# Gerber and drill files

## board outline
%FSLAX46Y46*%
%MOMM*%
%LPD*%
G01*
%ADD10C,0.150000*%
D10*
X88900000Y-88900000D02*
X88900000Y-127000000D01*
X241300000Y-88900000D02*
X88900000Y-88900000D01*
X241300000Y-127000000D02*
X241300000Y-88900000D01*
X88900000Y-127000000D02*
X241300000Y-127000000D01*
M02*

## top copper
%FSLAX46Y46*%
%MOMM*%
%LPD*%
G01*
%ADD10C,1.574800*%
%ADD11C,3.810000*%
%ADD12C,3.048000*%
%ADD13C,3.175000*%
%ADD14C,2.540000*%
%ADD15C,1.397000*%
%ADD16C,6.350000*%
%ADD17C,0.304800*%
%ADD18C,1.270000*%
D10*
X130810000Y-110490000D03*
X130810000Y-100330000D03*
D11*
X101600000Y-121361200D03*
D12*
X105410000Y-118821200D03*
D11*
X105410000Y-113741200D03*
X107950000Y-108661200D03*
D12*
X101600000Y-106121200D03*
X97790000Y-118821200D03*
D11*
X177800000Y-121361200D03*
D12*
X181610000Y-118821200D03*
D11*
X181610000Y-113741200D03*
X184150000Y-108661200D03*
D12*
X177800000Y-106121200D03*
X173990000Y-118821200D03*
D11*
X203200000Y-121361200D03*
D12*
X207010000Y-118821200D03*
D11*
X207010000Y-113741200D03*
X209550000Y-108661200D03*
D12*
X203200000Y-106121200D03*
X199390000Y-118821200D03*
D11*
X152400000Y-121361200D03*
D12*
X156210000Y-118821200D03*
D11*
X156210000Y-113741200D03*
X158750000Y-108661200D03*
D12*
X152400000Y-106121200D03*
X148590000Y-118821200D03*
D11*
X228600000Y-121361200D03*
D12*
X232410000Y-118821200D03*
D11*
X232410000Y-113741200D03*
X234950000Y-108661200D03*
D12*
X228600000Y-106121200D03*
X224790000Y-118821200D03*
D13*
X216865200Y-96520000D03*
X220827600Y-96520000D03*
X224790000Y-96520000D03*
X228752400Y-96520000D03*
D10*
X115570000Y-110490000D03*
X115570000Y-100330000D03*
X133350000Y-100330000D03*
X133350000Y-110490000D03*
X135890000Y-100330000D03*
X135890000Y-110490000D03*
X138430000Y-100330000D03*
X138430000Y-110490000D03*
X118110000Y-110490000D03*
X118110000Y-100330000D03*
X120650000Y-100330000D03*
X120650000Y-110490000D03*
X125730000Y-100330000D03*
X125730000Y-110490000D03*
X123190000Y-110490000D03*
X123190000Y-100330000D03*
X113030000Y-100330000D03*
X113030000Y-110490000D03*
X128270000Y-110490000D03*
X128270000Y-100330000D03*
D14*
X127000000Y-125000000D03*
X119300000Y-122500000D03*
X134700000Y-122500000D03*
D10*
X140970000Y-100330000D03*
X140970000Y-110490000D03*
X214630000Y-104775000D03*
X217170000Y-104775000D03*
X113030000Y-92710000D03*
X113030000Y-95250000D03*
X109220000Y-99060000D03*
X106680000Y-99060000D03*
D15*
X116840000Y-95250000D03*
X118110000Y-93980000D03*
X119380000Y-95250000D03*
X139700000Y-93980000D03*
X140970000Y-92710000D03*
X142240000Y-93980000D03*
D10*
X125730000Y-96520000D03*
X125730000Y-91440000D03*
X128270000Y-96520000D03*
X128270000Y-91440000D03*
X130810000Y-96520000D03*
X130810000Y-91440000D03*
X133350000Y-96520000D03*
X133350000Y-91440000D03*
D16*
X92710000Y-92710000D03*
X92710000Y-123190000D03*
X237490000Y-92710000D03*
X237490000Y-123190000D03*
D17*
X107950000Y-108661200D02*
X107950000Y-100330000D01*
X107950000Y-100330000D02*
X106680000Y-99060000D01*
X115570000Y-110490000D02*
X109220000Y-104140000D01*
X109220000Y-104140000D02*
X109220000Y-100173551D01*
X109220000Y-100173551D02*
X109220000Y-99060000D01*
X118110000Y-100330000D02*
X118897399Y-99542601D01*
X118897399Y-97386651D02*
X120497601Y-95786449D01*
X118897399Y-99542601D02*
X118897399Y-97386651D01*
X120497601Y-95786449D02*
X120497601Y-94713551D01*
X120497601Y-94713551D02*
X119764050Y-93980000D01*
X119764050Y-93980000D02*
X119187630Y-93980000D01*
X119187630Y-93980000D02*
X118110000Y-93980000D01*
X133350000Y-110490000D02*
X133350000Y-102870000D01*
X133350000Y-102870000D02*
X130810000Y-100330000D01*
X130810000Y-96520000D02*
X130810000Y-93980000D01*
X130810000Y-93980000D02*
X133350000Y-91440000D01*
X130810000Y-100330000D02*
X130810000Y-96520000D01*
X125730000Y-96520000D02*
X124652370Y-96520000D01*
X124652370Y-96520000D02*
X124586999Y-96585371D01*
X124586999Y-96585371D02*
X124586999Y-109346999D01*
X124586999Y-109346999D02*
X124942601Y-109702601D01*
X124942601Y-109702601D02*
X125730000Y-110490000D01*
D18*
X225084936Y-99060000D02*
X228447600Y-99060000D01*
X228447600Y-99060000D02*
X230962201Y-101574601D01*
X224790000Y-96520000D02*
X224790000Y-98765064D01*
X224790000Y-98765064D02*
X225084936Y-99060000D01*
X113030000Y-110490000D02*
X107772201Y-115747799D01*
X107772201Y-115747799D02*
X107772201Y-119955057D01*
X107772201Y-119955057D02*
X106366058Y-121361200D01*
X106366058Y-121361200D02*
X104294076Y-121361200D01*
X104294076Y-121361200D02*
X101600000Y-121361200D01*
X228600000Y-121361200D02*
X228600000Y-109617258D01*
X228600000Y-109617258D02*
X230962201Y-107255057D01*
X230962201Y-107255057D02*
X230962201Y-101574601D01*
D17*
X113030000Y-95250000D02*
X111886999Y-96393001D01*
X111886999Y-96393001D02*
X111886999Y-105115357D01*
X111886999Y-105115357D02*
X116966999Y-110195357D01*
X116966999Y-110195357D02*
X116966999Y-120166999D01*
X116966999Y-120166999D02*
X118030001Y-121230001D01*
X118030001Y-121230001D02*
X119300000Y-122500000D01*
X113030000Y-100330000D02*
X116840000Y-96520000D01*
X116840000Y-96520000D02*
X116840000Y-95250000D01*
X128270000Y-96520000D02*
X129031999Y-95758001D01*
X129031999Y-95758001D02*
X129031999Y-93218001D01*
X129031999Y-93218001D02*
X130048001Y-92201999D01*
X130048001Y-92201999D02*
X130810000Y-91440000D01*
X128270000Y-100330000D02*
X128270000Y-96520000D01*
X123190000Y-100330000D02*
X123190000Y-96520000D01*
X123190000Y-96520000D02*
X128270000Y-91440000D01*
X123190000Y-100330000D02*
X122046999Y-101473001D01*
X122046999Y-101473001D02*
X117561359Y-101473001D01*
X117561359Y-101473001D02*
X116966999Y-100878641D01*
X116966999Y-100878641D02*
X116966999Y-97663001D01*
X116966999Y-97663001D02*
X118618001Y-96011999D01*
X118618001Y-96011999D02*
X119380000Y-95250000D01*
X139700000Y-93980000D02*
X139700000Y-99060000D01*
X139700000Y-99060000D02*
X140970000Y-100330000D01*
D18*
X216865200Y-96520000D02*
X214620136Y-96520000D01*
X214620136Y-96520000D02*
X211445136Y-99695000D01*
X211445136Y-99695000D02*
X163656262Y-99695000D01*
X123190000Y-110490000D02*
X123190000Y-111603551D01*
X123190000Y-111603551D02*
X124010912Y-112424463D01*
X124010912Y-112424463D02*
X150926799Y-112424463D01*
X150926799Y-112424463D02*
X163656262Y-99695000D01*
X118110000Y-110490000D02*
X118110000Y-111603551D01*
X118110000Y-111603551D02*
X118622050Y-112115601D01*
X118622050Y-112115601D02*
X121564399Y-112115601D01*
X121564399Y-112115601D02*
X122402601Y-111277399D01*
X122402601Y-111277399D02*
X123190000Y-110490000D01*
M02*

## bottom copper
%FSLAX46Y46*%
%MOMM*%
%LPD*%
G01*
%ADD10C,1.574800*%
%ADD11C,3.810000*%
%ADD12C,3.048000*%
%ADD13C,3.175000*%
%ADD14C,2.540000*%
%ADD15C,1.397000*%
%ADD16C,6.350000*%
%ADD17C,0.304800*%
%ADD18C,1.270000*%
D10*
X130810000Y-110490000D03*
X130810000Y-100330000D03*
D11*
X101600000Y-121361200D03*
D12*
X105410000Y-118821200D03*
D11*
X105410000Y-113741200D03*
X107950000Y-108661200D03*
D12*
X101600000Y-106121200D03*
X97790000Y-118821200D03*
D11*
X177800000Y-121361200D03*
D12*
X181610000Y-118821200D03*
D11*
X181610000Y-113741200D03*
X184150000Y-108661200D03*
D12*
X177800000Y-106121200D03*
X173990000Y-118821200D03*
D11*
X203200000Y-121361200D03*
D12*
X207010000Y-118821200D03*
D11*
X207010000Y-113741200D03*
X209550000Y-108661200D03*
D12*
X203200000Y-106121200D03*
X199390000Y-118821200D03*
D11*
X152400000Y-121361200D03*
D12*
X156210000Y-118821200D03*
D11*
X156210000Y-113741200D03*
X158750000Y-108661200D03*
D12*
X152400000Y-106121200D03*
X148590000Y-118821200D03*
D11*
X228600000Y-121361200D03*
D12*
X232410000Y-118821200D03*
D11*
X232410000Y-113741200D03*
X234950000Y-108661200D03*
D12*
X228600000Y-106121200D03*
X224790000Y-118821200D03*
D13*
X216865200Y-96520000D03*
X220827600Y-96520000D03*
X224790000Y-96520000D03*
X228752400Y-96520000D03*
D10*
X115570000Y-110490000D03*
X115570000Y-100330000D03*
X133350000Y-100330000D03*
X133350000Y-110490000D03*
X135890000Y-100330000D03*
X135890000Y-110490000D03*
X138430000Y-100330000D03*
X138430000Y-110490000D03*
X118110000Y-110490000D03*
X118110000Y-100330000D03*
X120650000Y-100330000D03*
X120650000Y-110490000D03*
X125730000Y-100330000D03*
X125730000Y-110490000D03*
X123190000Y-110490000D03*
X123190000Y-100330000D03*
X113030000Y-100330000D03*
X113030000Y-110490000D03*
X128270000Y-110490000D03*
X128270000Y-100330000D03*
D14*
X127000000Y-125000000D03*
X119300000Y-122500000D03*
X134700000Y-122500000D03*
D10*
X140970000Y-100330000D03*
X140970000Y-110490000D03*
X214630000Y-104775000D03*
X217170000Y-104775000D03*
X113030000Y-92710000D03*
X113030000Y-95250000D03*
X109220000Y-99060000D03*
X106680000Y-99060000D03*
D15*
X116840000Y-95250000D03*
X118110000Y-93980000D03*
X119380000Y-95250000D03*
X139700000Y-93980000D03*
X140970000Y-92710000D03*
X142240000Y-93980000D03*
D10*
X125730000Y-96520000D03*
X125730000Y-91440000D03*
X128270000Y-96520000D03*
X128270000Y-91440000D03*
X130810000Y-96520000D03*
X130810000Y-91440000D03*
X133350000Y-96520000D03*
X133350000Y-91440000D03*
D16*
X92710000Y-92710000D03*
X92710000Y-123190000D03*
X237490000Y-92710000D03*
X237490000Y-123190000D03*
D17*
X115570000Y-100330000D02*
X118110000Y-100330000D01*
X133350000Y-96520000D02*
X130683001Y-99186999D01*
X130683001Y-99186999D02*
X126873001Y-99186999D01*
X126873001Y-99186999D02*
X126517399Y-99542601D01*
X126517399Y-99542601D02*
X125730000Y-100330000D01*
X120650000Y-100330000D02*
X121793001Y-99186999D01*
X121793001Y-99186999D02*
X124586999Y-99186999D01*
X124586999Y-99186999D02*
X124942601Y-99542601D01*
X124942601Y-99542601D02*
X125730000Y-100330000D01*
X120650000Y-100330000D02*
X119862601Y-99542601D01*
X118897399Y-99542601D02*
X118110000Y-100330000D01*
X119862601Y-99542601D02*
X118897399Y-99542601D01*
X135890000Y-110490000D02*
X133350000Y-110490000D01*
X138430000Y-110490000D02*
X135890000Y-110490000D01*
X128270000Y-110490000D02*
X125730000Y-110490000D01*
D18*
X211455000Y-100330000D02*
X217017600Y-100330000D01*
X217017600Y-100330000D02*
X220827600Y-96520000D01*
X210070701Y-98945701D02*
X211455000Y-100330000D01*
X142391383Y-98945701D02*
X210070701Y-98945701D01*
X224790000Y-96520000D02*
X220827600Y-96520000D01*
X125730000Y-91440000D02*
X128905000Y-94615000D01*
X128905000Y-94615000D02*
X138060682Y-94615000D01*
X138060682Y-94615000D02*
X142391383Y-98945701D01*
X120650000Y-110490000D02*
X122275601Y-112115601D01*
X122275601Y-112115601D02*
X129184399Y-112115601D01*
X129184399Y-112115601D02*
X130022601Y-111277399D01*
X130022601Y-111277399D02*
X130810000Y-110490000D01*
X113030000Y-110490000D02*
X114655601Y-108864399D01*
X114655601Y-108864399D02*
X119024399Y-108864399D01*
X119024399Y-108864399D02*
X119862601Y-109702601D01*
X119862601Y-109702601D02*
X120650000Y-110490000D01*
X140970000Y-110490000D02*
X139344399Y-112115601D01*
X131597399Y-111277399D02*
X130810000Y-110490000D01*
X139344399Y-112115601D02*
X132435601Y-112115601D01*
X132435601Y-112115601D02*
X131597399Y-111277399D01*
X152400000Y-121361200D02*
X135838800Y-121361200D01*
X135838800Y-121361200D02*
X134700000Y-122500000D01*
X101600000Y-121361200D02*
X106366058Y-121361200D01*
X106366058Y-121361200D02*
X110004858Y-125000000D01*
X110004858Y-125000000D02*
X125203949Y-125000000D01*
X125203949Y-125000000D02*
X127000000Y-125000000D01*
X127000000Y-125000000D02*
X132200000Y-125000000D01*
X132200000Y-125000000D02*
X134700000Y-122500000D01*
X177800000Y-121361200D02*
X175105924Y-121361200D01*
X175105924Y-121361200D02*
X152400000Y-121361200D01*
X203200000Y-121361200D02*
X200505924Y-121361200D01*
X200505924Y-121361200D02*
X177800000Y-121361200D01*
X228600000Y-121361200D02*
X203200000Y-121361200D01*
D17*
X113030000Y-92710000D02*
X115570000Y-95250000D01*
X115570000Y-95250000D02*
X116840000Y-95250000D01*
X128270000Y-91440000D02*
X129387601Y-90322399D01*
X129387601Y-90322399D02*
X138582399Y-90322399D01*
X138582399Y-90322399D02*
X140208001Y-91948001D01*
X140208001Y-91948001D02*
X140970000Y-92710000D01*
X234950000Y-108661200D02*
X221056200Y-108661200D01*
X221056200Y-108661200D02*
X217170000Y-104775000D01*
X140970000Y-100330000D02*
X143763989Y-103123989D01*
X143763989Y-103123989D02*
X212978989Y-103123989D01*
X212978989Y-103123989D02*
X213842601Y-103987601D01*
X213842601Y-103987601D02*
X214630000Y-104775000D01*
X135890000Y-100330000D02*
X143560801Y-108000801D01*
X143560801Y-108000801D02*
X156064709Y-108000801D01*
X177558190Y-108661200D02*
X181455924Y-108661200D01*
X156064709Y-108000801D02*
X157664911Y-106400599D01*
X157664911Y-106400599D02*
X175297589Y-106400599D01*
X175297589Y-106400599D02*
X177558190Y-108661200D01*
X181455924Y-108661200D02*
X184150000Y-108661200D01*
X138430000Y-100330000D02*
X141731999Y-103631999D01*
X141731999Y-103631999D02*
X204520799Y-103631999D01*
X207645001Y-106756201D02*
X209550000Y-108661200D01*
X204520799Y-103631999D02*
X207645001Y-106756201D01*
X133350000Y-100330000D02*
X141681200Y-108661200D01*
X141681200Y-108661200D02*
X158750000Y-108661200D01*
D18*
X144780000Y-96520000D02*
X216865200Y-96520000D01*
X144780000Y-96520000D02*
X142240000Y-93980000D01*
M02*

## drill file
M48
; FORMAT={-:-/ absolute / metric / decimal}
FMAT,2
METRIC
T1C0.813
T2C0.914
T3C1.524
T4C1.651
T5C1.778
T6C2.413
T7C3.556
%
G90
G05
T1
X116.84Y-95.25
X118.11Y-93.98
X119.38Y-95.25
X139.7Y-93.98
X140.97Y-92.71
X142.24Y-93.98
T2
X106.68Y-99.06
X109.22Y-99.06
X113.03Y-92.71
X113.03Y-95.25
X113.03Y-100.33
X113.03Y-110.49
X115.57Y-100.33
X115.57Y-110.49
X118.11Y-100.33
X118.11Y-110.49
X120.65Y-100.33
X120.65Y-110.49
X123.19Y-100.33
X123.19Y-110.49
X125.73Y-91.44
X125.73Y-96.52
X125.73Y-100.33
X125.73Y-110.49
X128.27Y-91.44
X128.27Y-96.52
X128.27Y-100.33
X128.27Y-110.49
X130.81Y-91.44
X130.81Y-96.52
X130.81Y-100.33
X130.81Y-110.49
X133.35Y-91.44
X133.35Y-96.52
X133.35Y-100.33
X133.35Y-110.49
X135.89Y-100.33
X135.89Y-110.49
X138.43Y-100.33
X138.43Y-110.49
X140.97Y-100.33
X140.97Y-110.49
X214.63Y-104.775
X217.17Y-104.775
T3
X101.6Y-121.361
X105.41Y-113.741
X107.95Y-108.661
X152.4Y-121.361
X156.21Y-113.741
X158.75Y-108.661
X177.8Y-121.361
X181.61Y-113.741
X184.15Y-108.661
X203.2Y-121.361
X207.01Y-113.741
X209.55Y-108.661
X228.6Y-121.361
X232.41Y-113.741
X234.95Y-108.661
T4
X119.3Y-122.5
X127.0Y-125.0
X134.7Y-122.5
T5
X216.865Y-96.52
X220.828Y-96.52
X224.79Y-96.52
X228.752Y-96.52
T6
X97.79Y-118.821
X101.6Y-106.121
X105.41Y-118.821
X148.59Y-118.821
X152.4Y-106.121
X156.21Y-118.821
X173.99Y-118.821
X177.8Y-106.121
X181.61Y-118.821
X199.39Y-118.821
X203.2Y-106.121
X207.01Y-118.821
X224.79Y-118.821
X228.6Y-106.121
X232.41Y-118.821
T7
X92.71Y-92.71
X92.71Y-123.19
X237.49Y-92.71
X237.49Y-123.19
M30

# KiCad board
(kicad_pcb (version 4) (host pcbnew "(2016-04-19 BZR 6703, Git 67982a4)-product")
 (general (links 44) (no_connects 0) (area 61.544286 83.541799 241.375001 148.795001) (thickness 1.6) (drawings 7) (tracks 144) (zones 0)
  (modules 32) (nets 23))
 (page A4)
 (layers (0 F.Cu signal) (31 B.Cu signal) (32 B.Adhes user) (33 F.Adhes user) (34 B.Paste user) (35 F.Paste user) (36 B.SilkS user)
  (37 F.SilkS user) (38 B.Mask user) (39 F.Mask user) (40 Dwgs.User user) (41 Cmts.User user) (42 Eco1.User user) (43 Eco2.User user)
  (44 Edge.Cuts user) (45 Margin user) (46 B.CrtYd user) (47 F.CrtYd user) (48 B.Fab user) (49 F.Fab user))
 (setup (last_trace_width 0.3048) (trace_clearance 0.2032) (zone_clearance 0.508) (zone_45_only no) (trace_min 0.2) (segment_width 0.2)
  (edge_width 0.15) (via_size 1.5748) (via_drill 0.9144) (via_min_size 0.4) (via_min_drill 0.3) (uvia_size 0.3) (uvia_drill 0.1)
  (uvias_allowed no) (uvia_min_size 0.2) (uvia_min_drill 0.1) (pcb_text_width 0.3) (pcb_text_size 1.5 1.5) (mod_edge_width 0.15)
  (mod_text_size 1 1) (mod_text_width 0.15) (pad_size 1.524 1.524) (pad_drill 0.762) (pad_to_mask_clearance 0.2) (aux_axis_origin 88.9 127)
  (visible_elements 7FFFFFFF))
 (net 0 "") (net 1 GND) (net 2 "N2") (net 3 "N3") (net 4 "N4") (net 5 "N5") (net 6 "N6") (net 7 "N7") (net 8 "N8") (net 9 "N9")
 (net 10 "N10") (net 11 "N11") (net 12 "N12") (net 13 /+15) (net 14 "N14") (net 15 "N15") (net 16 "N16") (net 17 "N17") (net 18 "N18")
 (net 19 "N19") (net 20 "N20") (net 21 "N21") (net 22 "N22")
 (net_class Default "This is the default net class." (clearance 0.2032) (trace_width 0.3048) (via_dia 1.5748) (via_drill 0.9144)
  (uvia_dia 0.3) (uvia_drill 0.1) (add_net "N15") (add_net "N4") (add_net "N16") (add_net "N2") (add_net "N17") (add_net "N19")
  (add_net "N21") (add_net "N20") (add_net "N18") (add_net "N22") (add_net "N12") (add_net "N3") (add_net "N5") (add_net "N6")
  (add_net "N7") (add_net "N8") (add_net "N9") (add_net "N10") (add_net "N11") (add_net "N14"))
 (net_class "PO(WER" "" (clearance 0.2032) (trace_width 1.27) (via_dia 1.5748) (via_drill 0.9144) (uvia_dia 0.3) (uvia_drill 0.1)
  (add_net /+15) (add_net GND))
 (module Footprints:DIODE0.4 (layer F.Cu) (at 130.81 105.41 90)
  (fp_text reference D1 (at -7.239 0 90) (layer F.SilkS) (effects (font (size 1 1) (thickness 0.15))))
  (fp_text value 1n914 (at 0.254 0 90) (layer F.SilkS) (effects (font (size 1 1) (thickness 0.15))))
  (pad 1 thru_hole circle (at -5.08 0 90) (size 1.5748 1.5748) (drill 0.9144) (layers *.Cu *.Mask F.SilkS) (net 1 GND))
  (pad 2 thru_hole circle (at 5.08 0 90) (size 1.5748 1.5748) (drill 0.9144) (layers *.Cu *.Mask F.SilkS) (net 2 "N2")))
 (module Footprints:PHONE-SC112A (layer F.Cu) (at 101.6 127 270)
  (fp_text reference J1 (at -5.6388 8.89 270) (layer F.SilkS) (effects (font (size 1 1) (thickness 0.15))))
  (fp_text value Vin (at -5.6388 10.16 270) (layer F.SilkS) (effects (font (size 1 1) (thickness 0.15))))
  (pad 1 thru_hole circle (at -5.6388 0 270) (size 3.81 3.81) (drill 1.524) (layers *.Cu *.Mask F.SilkS) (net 1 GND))
  (pad "" thru_hole circle (at -8.1788 -3.81 270) (size 3.048 3.048) (drill 2.413) (layers *.Cu *.Mask F.SilkS))
  (pad 2 thru_hole circle (at -13.2588 -3.81 270) (size 3.81 3.81) (drill 1.524) (layers *.Cu *.Mask F.SilkS) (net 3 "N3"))
  (pad 3 thru_hole circle (at -18.3388 -6.35 270) (size 3.81 3.81) (drill 1.524) (layers *.Cu *.Mask F.SilkS) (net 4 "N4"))
  (pad "" thru_hole circle (at -20.8788 0 270) (size 3.048 3.048) (drill 2.413) (layers *.Cu *.Mask F.SilkS))
  (pad "" thru_hole circle (at -8.1788 3.81 270) (size 3.048 3.048) (drill 2.413) (layers *.Cu *.Mask F.SilkS)))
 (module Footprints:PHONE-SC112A (layer F.Cu) (at 177.8 127 270)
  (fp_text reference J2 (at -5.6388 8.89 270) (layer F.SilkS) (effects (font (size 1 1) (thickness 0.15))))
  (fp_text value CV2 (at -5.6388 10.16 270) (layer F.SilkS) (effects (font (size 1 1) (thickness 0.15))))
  (pad 1 thru_hole circle (at -5.6388 0 270) (size 3.81 3.81) (drill 1.524) (layers *.Cu *.Mask F.SilkS) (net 1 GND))
  (pad "" thru_hole circle (at -8.1788 -3.81 270) (size 3.048 3.048) (drill 2.413) (layers *.Cu *.Mask F.SilkS))
  (pad 2 thru_hole circle (at -13.2588 -3.81 270) (size 3.81 3.81) (drill 1.524) (layers *.Cu *.Mask F.SilkS) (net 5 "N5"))
  (pad 3 thru_hole circle (at -18.3388 -6.35 270) (size 3.81 3.81) (drill 1.524) (layers *.Cu *.Mask F.SilkS) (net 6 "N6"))
  (pad "" thru_hole circle (at -20.8788 0 270) (size 3.048 3.048) (drill 2.413) (layers *.Cu *.Mask F.SilkS))
  (pad "" thru_hole circle (at -8.1788 3.81 270) (size 3.048 3.048) (drill 2.413) (layers *.Cu *.Mask F.SilkS)))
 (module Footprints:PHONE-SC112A (layer F.Cu) (at 203.2 127 270)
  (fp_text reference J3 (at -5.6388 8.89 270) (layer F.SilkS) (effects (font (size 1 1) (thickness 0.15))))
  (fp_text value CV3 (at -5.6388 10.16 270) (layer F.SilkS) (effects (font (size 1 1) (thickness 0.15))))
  (pad 1 thru_hole circle (at -5.6388 0 270) (size 3.81 3.81) (drill 1.524) (layers *.Cu *.Mask F.SilkS) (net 1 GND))
  (pad "" thru_hole circle (at -8.1788 -3.81 270) (size 3.048 3.048) (drill 2.413) (layers *.Cu *.Mask F.SilkS))
  (pad 2 thru_hole circle (at -13.2588 -3.81 270) (size 3.81 3.81) (drill 1.524) (layers *.Cu *.Mask F.SilkS) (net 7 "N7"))
  (pad 3 thru_hole circle (at -18.3388 -6.35 270) (size 3.81 3.81) (drill 1.524) (layers *.Cu *.Mask F.SilkS) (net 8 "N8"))
  (pad "" thru_hole circle (at -20.8788 0 270) (size 3.048 3.048) (drill 2.413) (layers *.Cu *.Mask F.SilkS))
  (pad "" thru_hole circle (at -8.1788 3.81 270) (size 3.048 3.048) (drill 2.413) (layers *.Cu *.Mask F.SilkS)))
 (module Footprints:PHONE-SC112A (layer F.Cu) (at 152.4 127 270)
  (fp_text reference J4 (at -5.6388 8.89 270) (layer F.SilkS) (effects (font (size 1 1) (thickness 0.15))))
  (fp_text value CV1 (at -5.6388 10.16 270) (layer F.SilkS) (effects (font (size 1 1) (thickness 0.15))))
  (pad 1 thru_hole circle (at -5.6388 0 270) (size 3.81 3.81) (drill 1.524) (layers *.Cu *.Mask F.SilkS) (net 1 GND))
  (pad "" thru_hole circle (at -8.1788 -3.81 270) (size 3.048 3.048) (drill 2.413) (layers *.Cu *.Mask F.SilkS))
  (pad 2 thru_hole circle (at -13.2588 -3.81 270) (size 3.81 3.81) (drill 1.524) (layers *.Cu *.Mask F.SilkS) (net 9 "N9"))
  (pad 3 thru_hole circle (at -18.3388 -6.35 270) (size 3.81 3.81) (drill 1.524) (layers *.Cu *.Mask F.SilkS) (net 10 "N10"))
  (pad "" thru_hole circle (at -20.8788 0 270) (size 3.048 3.048) (drill 2.413) (layers *.Cu *.Mask F.SilkS))
  (pad "" thru_hole circle (at -8.1788 3.81 270) (size 3.048 3.048) (drill 2.413) (layers *.Cu *.Mask F.SilkS)))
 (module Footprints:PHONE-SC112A (layer F.Cu) (at 228.6 127 270)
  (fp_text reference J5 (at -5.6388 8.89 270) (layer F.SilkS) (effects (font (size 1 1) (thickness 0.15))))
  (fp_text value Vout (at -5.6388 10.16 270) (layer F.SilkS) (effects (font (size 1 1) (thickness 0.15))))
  (pad 1 thru_hole circle (at -5.6388 0 270) (size 3.81 3.81) (drill 1.524) (layers *.Cu *.Mask F.SilkS) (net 1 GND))
  (pad "" thru_hole circle (at -8.1788 -3.81 270) (size 3.048 3.048) (drill 2.413) (layers *.Cu *.Mask F.SilkS))
  (pad 2 thru_hole circle (at -13.2588 -3.81 270) (size 3.81 3.81) (drill 1.524) (layers *.Cu *.Mask F.SilkS) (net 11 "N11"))
  (pad 3 thru_hole circle (at -18.3388 -6.35 270) (size 3.81 3.81) (drill 1.524) (layers *.Cu *.Mask F.SilkS) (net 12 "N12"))
  (pad "" thru_hole circle (at -20.8788 0 270) (size 3.048 3.048) (drill 2.413) (layers *.Cu *.Mask F.SilkS))
  (pad "" thru_hole circle (at -8.1788 3.81 270) (size 3.048 3.048) (drill 2.413) (layers *.Cu *.Mask F.SilkS)))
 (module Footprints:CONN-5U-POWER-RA (layer F.Cu) (at 222.8088 96.52)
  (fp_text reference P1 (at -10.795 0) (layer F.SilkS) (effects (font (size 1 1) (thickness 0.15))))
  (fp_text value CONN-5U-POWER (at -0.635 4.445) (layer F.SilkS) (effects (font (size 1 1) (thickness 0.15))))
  (pad 1 thru_hole circle (at -5.9436 0) (size 3.175 3.175) (drill 1.778) (layers *.Cu *.Mask F.SilkS) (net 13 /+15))
  (pad 2 thru_hole circle (at -1.9812 0) (size 3.175 3.175) (drill 1.778) (layers *.Cu *.Mask F.SilkS) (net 1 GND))
  (pad 3 thru_hole circle (at 1.9812 0) (size 3.175 3.175) (drill 1.778) (layers *.Cu *.Mask F.SilkS) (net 1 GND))
  (pad 4 thru_hole circle (at 5.9436 0) (size 3.175 3.175) (drill 1.778) (layers *.Cu *.Mask F.SilkS) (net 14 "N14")))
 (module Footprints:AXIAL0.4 (layer F.Cu) (at 115.57 105.41 90)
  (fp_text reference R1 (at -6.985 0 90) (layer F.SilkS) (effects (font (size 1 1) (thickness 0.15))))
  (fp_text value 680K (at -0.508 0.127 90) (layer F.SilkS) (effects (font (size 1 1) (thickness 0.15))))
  (pad 1 thru_hole circle (at -5.08 0 90) (size 1.5748 1.5748) (drill 0.9144) (layers *.Cu *.Mask F.SilkS) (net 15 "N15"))
  (pad 2 thru_hole circle (at 5.08 0 90) (size 1.5748 1.5748) (drill 0.9144) (layers *.Cu *.Mask F.SilkS) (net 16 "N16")))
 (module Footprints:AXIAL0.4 (layer F.Cu) (at 133.35 105.41 270)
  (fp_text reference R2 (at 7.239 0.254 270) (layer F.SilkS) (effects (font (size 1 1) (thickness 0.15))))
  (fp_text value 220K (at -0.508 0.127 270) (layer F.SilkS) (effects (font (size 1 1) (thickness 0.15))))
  (pad 1 thru_hole circle (at -5.08 0 270) (size 1.5748 1.5748) (drill 0.9144) (layers *.Cu *.Mask F.SilkS) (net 10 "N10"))
  (pad 2 thru_hole circle (at 5.08 0 270) (size 1.5748 1.5748) (drill 0.9144) (layers *.Cu *.Mask F.SilkS) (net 2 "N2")))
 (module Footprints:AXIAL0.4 (layer F.Cu) (at 135.89 105.41 270)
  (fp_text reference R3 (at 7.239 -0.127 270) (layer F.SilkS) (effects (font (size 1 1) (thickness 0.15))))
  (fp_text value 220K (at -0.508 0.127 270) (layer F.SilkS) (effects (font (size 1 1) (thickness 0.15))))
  (pad 1 thru_hole circle (at -5.08 0 270) (size 1.5748 1.5748) (drill 0.9144) (layers *.Cu *.Mask F.SilkS) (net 6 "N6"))
  (pad 2 thru_hole circle (at 5.08 0 270) (size 1.5748 1.5748) (drill 0.9144) (layers *.Cu *.Mask F.SilkS) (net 2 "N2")))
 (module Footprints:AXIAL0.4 (layer F.Cu) (at 138.43 105.41 270)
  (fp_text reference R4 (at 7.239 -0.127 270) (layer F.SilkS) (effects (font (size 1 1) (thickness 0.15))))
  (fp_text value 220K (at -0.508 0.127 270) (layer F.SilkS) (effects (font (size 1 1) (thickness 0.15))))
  (pad 1 thru_hole circle (at -5.08 0 270) (size 1.5748 1.5748) (drill 0.9144) (layers *.Cu *.Mask F.SilkS) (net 8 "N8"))
  (pad 2 thru_hole circle (at 5.08 0 270) (size 1.5748 1.5748) (drill 0.9144) (layers *.Cu *.Mask F.SilkS) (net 2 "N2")))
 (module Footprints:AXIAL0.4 (layer F.Cu) (at 118.11 105.41 90)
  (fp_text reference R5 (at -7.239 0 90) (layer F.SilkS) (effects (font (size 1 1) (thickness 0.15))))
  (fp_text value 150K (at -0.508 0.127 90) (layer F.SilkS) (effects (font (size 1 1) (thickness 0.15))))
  (pad 1 thru_hole circle (at -5.08 0 90) (size 1.5748 1.5748) (drill 0.9144) (layers *.Cu *.Mask F.SilkS) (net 13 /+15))
  (pad 2 thru_hole circle (at 5.08 0 90) (size 1.5748 1.5748) (drill 0.9144) (layers *.Cu *.Mask F.SilkS) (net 16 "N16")))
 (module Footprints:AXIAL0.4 (layer F.Cu) (at 120.65 105.41 270)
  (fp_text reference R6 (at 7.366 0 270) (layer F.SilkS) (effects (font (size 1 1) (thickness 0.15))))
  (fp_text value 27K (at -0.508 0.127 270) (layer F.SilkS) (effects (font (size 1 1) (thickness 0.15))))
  (pad 1 thru_hole circle (at -5.08 0 270) (size 1.5748 1.5748) (drill 0.9144) (layers *.Cu *.Mask F.SilkS) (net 16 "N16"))
  (pad 2 thru_hole circle (at 5.08 0 270) (size 1.5748 1.5748) (drill 0.9144) (layers *.Cu *.Mask F.SilkS) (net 1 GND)))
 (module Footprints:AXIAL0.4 (layer F.Cu) (at 125.73 105.41 270)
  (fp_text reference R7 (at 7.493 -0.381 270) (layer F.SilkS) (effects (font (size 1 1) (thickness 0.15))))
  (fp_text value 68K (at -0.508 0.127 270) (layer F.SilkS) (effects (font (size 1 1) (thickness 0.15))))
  (pad 1 thru_hole circle (at -5.08 0 270) (size 1.5748 1.5748) (drill 0.9144) (layers *.Cu *.Mask F.SilkS) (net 16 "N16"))
  (pad 2 thru_hole circle (at 5.08 0 270) (size 1.5748 1.5748) (drill 0.9144) (layers *.Cu *.Mask F.SilkS) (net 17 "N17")))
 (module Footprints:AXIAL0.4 (layer F.Cu) (at 123.19 105.41 90)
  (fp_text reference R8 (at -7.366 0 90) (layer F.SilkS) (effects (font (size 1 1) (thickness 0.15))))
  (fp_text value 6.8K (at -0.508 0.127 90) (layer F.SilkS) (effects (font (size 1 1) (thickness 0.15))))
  (pad 1 thru_hole circle (at -5.08 0 90) (size 1.5748 1.5748) (drill 0.9144) (layers *.Cu *.Mask F.SilkS) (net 13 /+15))
  (pad 2 thru_hole circle (at 5.08 0 90) (size 1.5748 1.5748) (drill 0.9144) (layers *.Cu *.Mask F.SilkS) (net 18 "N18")))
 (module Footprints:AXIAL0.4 (layer F.Cu) (at 113.03 105.41 270)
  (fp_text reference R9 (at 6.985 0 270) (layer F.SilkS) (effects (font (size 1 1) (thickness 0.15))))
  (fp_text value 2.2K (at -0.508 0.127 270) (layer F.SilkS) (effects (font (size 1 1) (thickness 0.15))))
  (pad 1 thru_hole circle (at -5.08 0 270) (size 1.5748 1.5748) (drill 0.9144) (layers *.Cu *.Mask F.SilkS) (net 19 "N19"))
  (pad 2 thru_hole circle (at 5.08 0 270) (size 1.5748 1.5748) (drill 0.9144) (layers *.Cu *.Mask F.SilkS) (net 1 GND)))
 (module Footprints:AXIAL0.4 (layer F.Cu) (at 128.27 105.41 90)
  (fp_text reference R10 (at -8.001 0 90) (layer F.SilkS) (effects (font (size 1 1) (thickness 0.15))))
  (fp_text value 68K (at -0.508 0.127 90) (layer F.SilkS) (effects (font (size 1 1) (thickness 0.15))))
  (pad 1 thru_hole circle (at -5.08 0 90) (size 1.5748 1.5748) (drill 0.9144) (layers *.Cu *.Mask F.SilkS) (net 17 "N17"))
  (pad 2 thru_hole circle (at 5.08 0 90) (size 1.5748 1.5748) (drill 0.9144) (layers *.Cu *.Mask F.SilkS) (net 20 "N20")))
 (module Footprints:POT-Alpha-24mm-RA (layer F.Cu) (at 127 127)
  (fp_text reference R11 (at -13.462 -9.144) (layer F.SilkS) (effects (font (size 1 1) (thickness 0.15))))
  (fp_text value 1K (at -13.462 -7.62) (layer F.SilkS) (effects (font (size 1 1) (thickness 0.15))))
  (pad 2 thru_hole circle (at 0 -2) (size 2.54 2.54) (drill 1.651) (layers *.Cu *.Mask F.SilkS) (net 1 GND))
  (pad 1 thru_hole circle (at -7.7 -4.5) (size 2.54 2.54) (drill 1.651) (layers *.Cu *.Mask F.SilkS) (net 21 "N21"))
  (pad 3 thru_hole circle (at 7.7 -4.5) (size 2.54 2.54) (drill 1.651) (layers *.Cu *.Mask F.SilkS) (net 1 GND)))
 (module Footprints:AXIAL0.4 (layer F.Cu) (at 140.97 105.41 270)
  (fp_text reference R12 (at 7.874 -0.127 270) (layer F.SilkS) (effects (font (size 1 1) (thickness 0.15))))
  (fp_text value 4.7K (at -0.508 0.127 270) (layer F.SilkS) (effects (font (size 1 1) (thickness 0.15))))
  (pad 1 thru_hole circle (at -5.08 0 270) (size 1.5748 1.5748) (drill 0.9144) (layers *.Cu *.Mask F.SilkS) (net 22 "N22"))
  (pad 2 thru_hole circle (at 5.08 0 270) (size 1.5748 1.5748) (drill 0.9144) (layers *.Cu *.Mask F.SilkS) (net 1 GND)))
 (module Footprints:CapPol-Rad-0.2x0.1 (layer F.Cu) (at 217.17 107.315)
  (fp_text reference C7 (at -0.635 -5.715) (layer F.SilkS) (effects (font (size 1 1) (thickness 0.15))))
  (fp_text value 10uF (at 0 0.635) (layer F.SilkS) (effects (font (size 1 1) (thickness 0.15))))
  (pad 1 thru_hole circle (at -2.54 -2.54) (size 1.5748 1.5748) (drill 0.9144) (layers *.Cu *.Mask F.SilkS) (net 22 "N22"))
  (pad 2 thru_hole circle (at 0 -2.54) (size 1.5748 1.5748) (drill 0.9144) (layers *.Cu *.Mask F.SilkS) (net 12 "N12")))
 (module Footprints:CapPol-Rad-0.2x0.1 (layer F.Cu) (at 110.49 95.25 270)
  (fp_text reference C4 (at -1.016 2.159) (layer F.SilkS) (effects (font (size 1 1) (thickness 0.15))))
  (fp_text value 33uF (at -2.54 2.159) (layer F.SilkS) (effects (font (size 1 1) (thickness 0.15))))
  (pad 1 thru_hole circle (at -2.54 -2.54 270) (size 1.5748 1.5748) (drill 0.9144) (layers *.Cu *.Mask F.SilkS) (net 19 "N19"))
  (pad 2 thru_hole circle (at 0 -2.54 270) (size 1.5748 1.5748) (drill 0.9144) (layers *.Cu *.Mask F.SilkS) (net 21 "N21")))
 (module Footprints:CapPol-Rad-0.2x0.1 (layer F.Cu) (at 106.68 96.52 180)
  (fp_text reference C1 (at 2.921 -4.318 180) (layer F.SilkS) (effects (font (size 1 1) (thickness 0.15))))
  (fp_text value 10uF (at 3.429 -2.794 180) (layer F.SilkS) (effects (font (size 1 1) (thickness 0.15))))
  (pad 1 thru_hole circle (at -2.54 -2.54 180) (size 1.5748 1.5748) (drill 0.9144) (layers *.Cu *.Mask F.SilkS) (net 15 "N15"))
  (pad 2 thru_hole circle (at 0 -2.54 180) (size 1.5748 1.5748) (drill 0.9144) (layers *.Cu *.Mask F.SilkS) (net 4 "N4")))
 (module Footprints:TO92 (layer F.Cu) (at 118.11 97.79)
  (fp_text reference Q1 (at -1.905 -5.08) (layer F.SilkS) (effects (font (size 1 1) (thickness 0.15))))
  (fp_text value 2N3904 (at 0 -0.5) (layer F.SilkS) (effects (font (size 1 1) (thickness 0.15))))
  (pad 1 thru_hole circle (at -1.27 -2.54) (size 1.397 1.397) (drill 0.8128) (layers *.Cu *.Mask F.SilkS) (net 19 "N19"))
  (pad 2 thru_hole circle (at 0 -3.81) (size 1.397 1.397) (drill 0.8128) (layers *.Cu *.Mask F.SilkS) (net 16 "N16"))
  (pad 3 thru_hole circle (at 1.27 -2.54) (size 1.397 1.397) (drill 0.8128) (layers *.Cu *.Mask F.SilkS) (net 18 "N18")))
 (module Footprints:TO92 (layer F.Cu) (at 140.97 96.52)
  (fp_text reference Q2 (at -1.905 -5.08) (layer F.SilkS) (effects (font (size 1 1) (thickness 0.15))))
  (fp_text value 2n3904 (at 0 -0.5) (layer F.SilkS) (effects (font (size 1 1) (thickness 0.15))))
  (pad 1 thru_hole circle (at -1.27 -2.54) (size 1.397 1.397) (drill 0.8128) (layers *.Cu *.Mask F.SilkS) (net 22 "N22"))
  (pad 2 thru_hole circle (at 0 -3.81) (size 1.397 1.397) (drill 0.8128) (layers *.Cu *.Mask F.SilkS) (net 18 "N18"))
  (pad 3 thru_hole circle (at 1.27 -2.54) (size 1.397 1.397) (drill 0.8128) (layers *.Cu *.Mask F.SilkS) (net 13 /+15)))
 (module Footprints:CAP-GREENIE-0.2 (layer F.Cu) (at 125.73 93.98 90)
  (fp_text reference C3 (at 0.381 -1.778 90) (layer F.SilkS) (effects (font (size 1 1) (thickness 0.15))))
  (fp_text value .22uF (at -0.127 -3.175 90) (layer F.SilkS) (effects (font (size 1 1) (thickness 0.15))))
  (pad 1 thru_hole circle (at -2.54 0 90) (size 1.5748 1.5748) (drill 0.9144) (layers *.Cu *.Mask F.SilkS) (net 17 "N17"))
  (pad 2 thru_hole circle (at 2.54 0 90) (size 1.5748 1.5748) (drill 0.9144) (layers *.Cu *.Mask F.SilkS) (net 1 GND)))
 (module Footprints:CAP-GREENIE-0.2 (layer F.Cu) (at 128.27 93.98 90)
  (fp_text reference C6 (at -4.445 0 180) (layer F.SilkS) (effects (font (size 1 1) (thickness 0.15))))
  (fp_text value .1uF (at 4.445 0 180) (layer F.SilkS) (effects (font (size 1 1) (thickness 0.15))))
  (pad 1 thru_hole circle (at -2.54 0 90) (size 1.5748 1.5748) (drill 0.9144) (layers *.Cu *.Mask F.SilkS) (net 20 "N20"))
  (pad 2 thru_hole circle (at 2.54 0 90) (size 1.5748 1.5748) (drill 0.9144) (layers *.Cu *.Mask F.SilkS) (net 18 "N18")))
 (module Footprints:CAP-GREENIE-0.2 (layer F.Cu) (at 130.81 93.98 90)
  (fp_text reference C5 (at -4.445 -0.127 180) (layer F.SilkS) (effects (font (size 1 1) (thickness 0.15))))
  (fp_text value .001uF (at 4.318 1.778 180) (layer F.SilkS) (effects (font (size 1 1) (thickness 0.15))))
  (pad 1 thru_hole circle (at -2.54 0 90) (size 1.5748 1.5748) (drill 0.9144) (layers *.Cu *.Mask F.SilkS) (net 2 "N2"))
  (pad 2 thru_hole circle (at 2.54 0 90) (size 1.5748 1.5748) (drill 0.9144) (layers *.Cu *.Mask F.SilkS) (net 20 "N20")))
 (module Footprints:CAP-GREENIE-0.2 (layer F.Cu) (at 133.35 93.98 90)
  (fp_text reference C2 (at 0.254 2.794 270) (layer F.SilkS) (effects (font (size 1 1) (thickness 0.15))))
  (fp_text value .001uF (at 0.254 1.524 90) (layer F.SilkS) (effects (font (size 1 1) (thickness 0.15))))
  (pad 1 thru_hole circle (at -2.54 0 90) (size 1.5748 1.5748) (drill 0.9144) (layers *.Cu *.Mask F.SilkS) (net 16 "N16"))
  (pad 2 thru_hole circle (at 2.54 0 90) (size 1.5748 1.5748) (drill 0.9144) (layers *.Cu *.Mask F.SilkS) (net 2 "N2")))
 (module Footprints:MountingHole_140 (layer F.Cu) (at 92.71 92.71)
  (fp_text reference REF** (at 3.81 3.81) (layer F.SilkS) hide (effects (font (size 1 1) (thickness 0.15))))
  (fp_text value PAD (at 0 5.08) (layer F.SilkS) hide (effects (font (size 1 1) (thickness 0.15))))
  (pad "" thru_hole circle (at 0 0) (size 6.35 6.35) (drill 3.556) (layers *.Cu *.Mask F.SilkS)))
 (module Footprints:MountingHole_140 (layer F.Cu) (at 92.71 123.19)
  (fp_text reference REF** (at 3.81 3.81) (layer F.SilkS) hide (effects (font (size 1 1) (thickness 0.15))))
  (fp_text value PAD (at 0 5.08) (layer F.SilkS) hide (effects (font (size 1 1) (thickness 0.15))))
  (pad "" thru_hole circle (at 0 0) (size 6.35 6.35) (drill 3.556) (layers *.Cu *.Mask F.SilkS)))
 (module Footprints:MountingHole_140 (layer F.Cu) (at 237.49 92.71)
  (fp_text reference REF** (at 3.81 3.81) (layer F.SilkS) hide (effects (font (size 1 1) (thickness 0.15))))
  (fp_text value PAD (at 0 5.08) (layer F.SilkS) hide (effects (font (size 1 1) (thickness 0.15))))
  (pad "" thru_hole circle (at 0 0) (size 6.35 6.35) (drill 3.556) (layers *.Cu *.Mask F.SilkS)))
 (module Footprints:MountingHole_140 (layer F.Cu) (at 237.49 123.19)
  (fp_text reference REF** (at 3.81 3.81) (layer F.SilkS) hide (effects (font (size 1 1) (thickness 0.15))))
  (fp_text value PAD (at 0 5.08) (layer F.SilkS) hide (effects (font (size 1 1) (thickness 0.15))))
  (pad "" thru_hole circle (at 0 0) (size 6.35 6.35) (drill 3.556) (layers *.Cu *.Mask F.SilkS)))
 (gr_line (start 88.9 88.9) (end 88.9 127) (layer Edge.Cuts) (width 0.15))
 (gr_line (start 241.3 88.9) (end 88.9 88.9) (layer Edge.Cuts) (width 0.15))
 (gr_line (start 241.3 127) (end 241.3 88.9) (layer Edge.Cuts) (width 0.15))
 (gr_line (start 88.9 127) (end 241.3 127) (layer Edge.Cuts) (width 0.15))
 (segment (start 107.95 108.6612) (end 107.95 100.33) (width 0.3048) (layer F.Cu) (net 4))
 (segment (start 107.95 100.33) (end 106.68 99.06) (width 0.3048) (layer F.Cu) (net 4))
 (segment (start 115.57 110.49) (end 109.22 104.14) (width 0.3048) (layer F.Cu) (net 15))
 (segment (start 109.22 104.14) (end 109.22 100.173551) (width 0.3048) (layer F.Cu) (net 15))
 (segment (start 109.22 100.173551) (end 109.22 99.06) (width 0.3048) (layer F.Cu) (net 15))
 (segment (start 115.57 100.33) (end 118.11 100.33) (width 0.3048) (layer B.Cu) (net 16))
 (segment (start 133.35 96.52) (end 130.683001 99.186999) (width 0.3048) (layer B.Cu) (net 16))
 (segment (start 130.683001 99.186999) (end 126.873001 99.186999) (width 0.3048) (layer B.Cu) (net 16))
 (segment (start 126.873001 99.186999) (end 126.517399 99.542601) (width 0.3048) (layer B.Cu) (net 16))
 (segment (start 126.517399 99.542601) (end 125.73 100.33) (width 0.3048) (layer B.Cu) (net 16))
 (segment (start 120.65 100.33) (end 121.793001 99.186999) (width 0.3048) (layer B.Cu) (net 16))
 (segment (start 121.793001 99.186999) (end 124.586999 99.186999) (width 0.3048) (layer B.Cu) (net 16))
 (segment (start 124.586999 99.186999) (end 124.942601 99.542601) (width 0.3048) (layer B.Cu) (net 16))
 (segment (start 124.942601 99.542601) (end 125.73 100.33) (width 0.3048) (layer B.Cu) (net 16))
 (segment (start 120.65 100.33) (end 119.862601 99.542601) (width 0.3048) (layer B.Cu) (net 16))
 (segment (start 118.897399 99.542601) (end 118.11 100.33) (width 0.3048) (layer B.Cu) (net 16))
 (segment (start 119.862601 99.542601) (end 118.897399 99.542601) (width 0.3048) (layer B.Cu) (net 16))
 (segment (start 118.11 100.33) (end 118.897399 99.542601) (width 0.3048) (layer F.Cu) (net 16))
 (segment (start 118.897399 97.386651) (end 120.497601 95.786449) (width 0.3048) (layer F.Cu) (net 16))
 (segment (start 118.897399 99.542601) (end 118.897399 97.386651) (width 0.3048) (layer F.Cu) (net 16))
 (segment (start 120.497601 95.786449) (end 120.497601 94.713551) (width 0.3048) (layer F.Cu) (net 16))
 (segment (start 120.497601 94.713551) (end 119.76405 93.98) (width 0.3048) (layer F.Cu) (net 16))
 (segment (start 119.76405 93.98) (end 119.18763 93.98) (width 0.3048) (layer F.Cu) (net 16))
 (segment (start 119.18763 93.98) (end 118.11 93.98) (width 0.3048) (layer F.Cu) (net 16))
 (segment (start 133.35 110.49) (end 133.35 102.87) (width 0.3048) (layer F.Cu) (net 2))
 (segment (start 133.35 102.87) (end 130.81 100.33) (width 0.3048) (layer F.Cu) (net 2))
 (segment (start 135.89 110.49) (end 133.35 110.49) (width 0.3048) (layer B.Cu) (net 2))
 (segment (start 138.43 110.49) (end 135.89 110.49) (width 0.3048) (layer B.Cu) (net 2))
 (segment (start 130.81 96.52) (end 130.81 93.98) (width 0.3048) (layer F.Cu) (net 2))
 (segment (start 130.81 93.98) (end 133.35 91.44) (width 0.3048) (layer F.Cu) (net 2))
 (segment (start 130.81 100.33) (end 130.81 96.52) (width 0.3048) (layer F.Cu) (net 2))
 (segment (start 128.27 110.49) (end 125.73 110.49) (width 0.3048) (layer B.Cu) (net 17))
 (segment (start 125.73 96.52) (end 124.65237 96.52) (width 0.3048) (layer F.Cu) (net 17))
 (segment (start 124.65237 96.52) (end 124.586999 96.585371) (width 0.3048) (layer F.Cu) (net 17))
 (segment (start 124.586999 96.585371) (end 124.586999 109.346999) (width 0.3048) (layer F.Cu) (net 17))
 (segment (start 124.586999 109.346999) (end 124.942601 109.702601) (width 0.3048) (layer F.Cu) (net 17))
 (segment (start 124.942601 109.702601) (end 125.73 110.49) (width 0.3048) (layer F.Cu) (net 17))
 (segment (start 211.455 100.33) (end 217.0176 100.33) (width 1.27) (layer B.Cu) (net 1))
 (segment (start 217.0176 100.33) (end 220.8276 96.52) (width 1.27) (layer B.Cu) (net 1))
 (segment (start 210.070701 98.945701) (end 211.455 100.33) (width 1.27) (layer B.Cu) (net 1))
 (segment (start 142.391383 98.945701) (end 210.070701 98.945701) (width 1.27) (layer B.Cu) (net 1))
 (segment (start 224.79 96.52) (end 220.8276 96.52) (width 1.27) (layer B.Cu) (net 1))
 (segment (start 225.084936 99.06) (end 228.4476 99.06) (width 1.27) (layer F.Cu) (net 1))
 (segment (start 228.4476 99.06) (end 230.962201 101.574601) (width 1.27) (layer F.Cu) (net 1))
 (segment (start 224.79 96.52) (end 224.79 98.765064) (width 1.27) (layer F.Cu) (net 1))
 (segment (start 224.79 98.765064) (end 225.084936 99.06) (width 1.27) (layer F.Cu) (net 1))
 (segment (start 125.73 91.44) (end 128.905 94.615) (width 1.27) (layer B.Cu) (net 1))
 (segment (start 128.905 94.615) (end 138.060682 94.615) (width 1.27) (layer B.Cu) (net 1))
 (segment (start 138.060682 94.615) (end 142.391383 98.945701) (width 1.27) (layer B.Cu) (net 1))
 (segment (start 113.03 110.49) (end 107.772201 115.747799) (width 1.27) (layer F.Cu) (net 1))
 (segment (start 107.772201 115.747799) (end 107.772201 119.955057) (width 1.27) (layer F.Cu) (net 1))
 (segment (start 107.772201 119.955057) (end 106.366058 121.3612) (width 1.27) (layer F.Cu) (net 1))
 (segment (start 106.366058 121.3612) (end 104.294076 121.3612) (width 1.27) (layer F.Cu) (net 1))
 (segment (start 104.294076 121.3612) (end 101.6 121.3612) (width 1.27) (layer F.Cu) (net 1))
 (segment (start 120.65 110.49) (end 122.275601 112.115601) (width 1.27) (layer B.Cu) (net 1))
 (segment (start 122.275601 112.115601) (end 129.184399 112.115601) (width 1.27) (layer B.Cu) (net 1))
 (segment (start 129.184399 112.115601) (end 130.022601 111.277399) (width 1.27) (layer B.Cu) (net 1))
 (segment (start 130.022601 111.277399) (end 130.81 110.49) (width 1.27) (layer B.Cu) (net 1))
 (segment (start 113.03 110.49) (end 114.655601 108.864399) (width 1.27) (layer B.Cu) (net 1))
 (segment (start 114.655601 108.864399) (end 119.024399 108.864399) (width 1.27) (layer B.Cu) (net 1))
 (segment (start 119.024399 108.864399) (end 119.862601 109.702601) (width 1.27) (layer B.Cu) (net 1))
 (segment (start 119.862601 109.702601) (end 120.65 110.49) (width 1.27) (layer B.Cu) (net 1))
 (segment (start 140.97 110.49) (end 139.344399 112.115601) (width 1.27) (layer B.Cu) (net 1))
 (segment (start 131.597399 111.277399) (end 130.81 110.49) (width 1.27) (layer B.Cu) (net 1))
 (segment (start 139.344399 112.115601) (end 132.435601 112.115601) (width 1.27) (layer B.Cu) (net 1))
 (segment (start 132.435601 112.115601) (end 131.597399 111.277399) (width 1.27) (layer B.Cu) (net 1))
 (segment (start 152.4 121.3612) (end 135.8388 121.3612) (width 1.27) (layer B.Cu) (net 1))
 (segment (start 135.8388 121.3612) (end 134.7 122.5) (width 1.27) (layer B.Cu) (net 1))
 (segment (start 101.6 121.3612) (end 106.366058 121.3612) (width 1.27) (layer B.Cu) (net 1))
 (segment (start 106.366058 121.3612) (end 110.004858 125) (width 1.27) (layer B.Cu) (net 1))
 (segment (start 110.004858 125) (end 125.203949 125) (width 1.27) (layer B.Cu) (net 1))
 (segment (start 125.203949 125) (end 127 125) (width 1.27) (layer B.Cu) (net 1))
 (segment (start 127 125) (end 132.2 125) (width 1.27) (layer B.Cu) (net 1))
 (segment (start 132.2 125) (end 134.7 122.5) (width 1.27) (layer B.Cu) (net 1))
 (segment (start 177.8 121.3612) (end 175.105924 121.3612) (width 1.27) (layer B.Cu) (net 1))
 (segment (start 175.105924 121.3612) (end 152.4 121.3612) (width 1.27) (layer B.Cu) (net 1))
 (segment (start 203.2 121.3612) (end 200.505924 121.3612) (width 1.27) (layer B.Cu) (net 1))
 (segment (start 200.505924 121.3612) (end 177.8 121.3612) (width 1.27) (layer B.Cu) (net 1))
 (segment (start 228.6 121.3612) (end 203.2 121.3612) (width 1.27) (layer B.Cu) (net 1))
 (segment (start 228.6 121.3612) (end 228.6 109.617258) (width 1.27) (layer F.Cu) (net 1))
 (segment (start 228.6 109.617258) (end 230.962201 107.255057) (width 1.27) (layer F.Cu) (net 1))
 (segment (start 230.962201 107.255057) (end 230.962201 101.574601) (width 1.27) (layer F.Cu) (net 1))
 (segment (start 113.03 95.25) (end 111.886999 96.393001) (width 0.3048) (layer F.Cu) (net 21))
 (segment (start 111.886999 96.393001) (end 111.886999 105.115357) (width 0.3048) (layer F.Cu) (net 21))
 (segment (start 111.886999 105.115357) (end 116.966999 110.195357) (width 0.3048) (layer F.Cu) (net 21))
 (segment (start 116.966999 110.195357) (end 116.966999 120.166999) (width 0.3048) (layer F.Cu) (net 21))
 (segment (start 116.966999 120.166999) (end 118.030001 121.230001) (width 0.3048) (layer F.Cu) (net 21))
 (segment (start 118.030001 121.230001) (end 119.3 122.5) (width 0.3048) (layer F.Cu) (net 21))
 (segment (start 113.03 92.71) (end 115.57 95.25) (width 0.3048) (layer B.Cu) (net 19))
 (segment (start 115.57 95.25) (end 116.84 95.25) (width 0.3048) (layer B.Cu) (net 19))
 (segment (start 113.03 100.33) (end 116.84 96.52) (width 0.3048) (layer F.Cu) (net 19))
 (segment (start 116.84 96.52) (end 116.84 95.25) (width 0.3048) (layer F.Cu) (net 19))
 (segment (start 128.27 96.52) (end 129.031999 95.758001) (width 0.3048) (layer F.Cu) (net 20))
 (segment (start 129.031999 95.758001) (end 129.031999 93.218001) (width 0.3048) (layer F.Cu) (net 20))
 (segment (start 129.031999 93.218001) (end 130.048001 92.201999) (width 0.3048) (layer F.Cu) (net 20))
 (segment (start 130.048001 92.201999) (end 130.81 91.44) (width 0.3048) (layer F.Cu) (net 20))
 (segment (start 128.27 100.33) (end 128.27 96.52) (width 0.3048) (layer F.Cu) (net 20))
 (segment (start 123.19 100.33) (end 123.19 96.52) (width 0.3048) (layer F.Cu) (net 18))
 (segment (start 123.19 96.52) (end 128.27 91.44) (width 0.3048) (layer F.Cu) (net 18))
 (segment (start 128.27 91.44) (end 129.387601 90.322399) (width 0.3048) (layer B.Cu) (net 18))
 (segment (start 129.387601 90.322399) (end 138.582399 90.322399) (width 0.3048) (layer B.Cu) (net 18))
 (segment (start 138.582399 90.322399) (end 140.208001 91.948001) (width 0.3048) (layer B.Cu) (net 18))
 (segment (start 140.208001 91.948001) (end 140.97 92.71) (width 0.3048) (layer B.Cu) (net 18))
 (segment (start 123.19 100.33) (end 122.046999 101.473001) (width 0.3048) (layer F.Cu) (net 18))
 (segment (start 122.046999 101.473001) (end 117.561359 101.473001) (width 0.3048) (layer F.Cu) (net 18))
 (segment (start 117.561359 101.473001) (end 116.966999 100.878641) (width 0.3048) (layer F.Cu) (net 18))
 (segment (start 116.966999 100.878641) (end 116.966999 97.663001) (width 0.3048) (layer F.Cu) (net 18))
 (segment (start 116.966999 97.663001) (end 118.618001 96.011999) (width 0.3048) (layer F.Cu) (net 18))
 (segment (start 118.618001 96.011999) (end 119.38 95.25) (width 0.3048) (layer F.Cu) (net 18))
 (segment (start 234.95 108.6612) (end 221.0562 108.6612) (width 0.3048) (layer B.Cu) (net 12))
 (segment (start 221.0562 108.6612) (end 217.17 104.775) (width 0.3048) (layer B.Cu) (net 12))
 (segment (start 140.97 100.33) (end 143.763989 103.123989) (width 0.3048) (layer B.Cu) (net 22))
 (segment (start 143.763989 103.123989) (end 212.978989 103.123989) (width 0.3048) (layer B.Cu) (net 22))
 (segment (start 212.978989 103.123989) (end 213.842601 103.987601) (width 0.3048) (layer B.Cu) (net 22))
 (segment (start 213.842601 103.987601) (end 214.63 104.775) (width 0.3048) (layer B.Cu) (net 22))
 (segment (start 139.7 93.98) (end 139.7 99.06) (width 0.3048) (layer F.Cu) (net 22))
 (segment (start 139.7 99.06) (end 140.97 100.33) (width 0.3048) (layer F.Cu) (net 22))
 (segment (start 135.89 100.33) (end 143.560801 108.000801) (width 0.3048) (layer B.Cu) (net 6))
 (segment (start 143.560801 108.000801) (end 156.064709 108.000801) (width 0.3048) (layer B.Cu) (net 6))
 (segment (start 177.55819 108.6612) (end 181.455924 108.6612) (width 0.3048) (layer B.Cu) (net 6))
 (segment (start 156.064709 108.000801) (end 157.664911 106.400599) (width 0.3048) (layer B.Cu) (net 6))
 (segment (start 157.664911 106.400599) (end 175.297589 106.400599) (width 0.3048) (layer B.Cu) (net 6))
 (segment (start 175.297589 106.400599) (end 177.55819 108.6612) (width 0.3048) (layer B.Cu) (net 6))
 (segment (start 181.455924 108.6612) (end 184.15 108.6612) (width 0.3048) (layer B.Cu) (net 6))
 (segment (start 138.43 100.33) (end 141.731999 103.631999) (width 0.3048) (layer B.Cu) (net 8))
 (segment (start 141.731999 103.631999) (end 204.520799 103.631999) (width 0.3048) (layer B.Cu) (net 8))
 (segment (start 207.645001 106.756201) (end 209.55 108.6612) (width 0.3048) (layer B.Cu) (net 8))
 (segment (start 204.520799 103.631999) (end 207.645001 106.756201) (width 0.3048) (layer B.Cu) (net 8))
 (segment (start 133.35 100.33) (end 141.6812 108.6612) (width 0.3048) (layer B.Cu) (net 10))
 (segment (start 141.6812 108.6612) (end 158.75 108.6612) (width 0.3048) (layer B.Cu) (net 10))
 (segment (start 144.78 96.52) (end 216.8652 96.52) (width 1.27) (layer B.Cu) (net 13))
 (segment (start 216.8652 96.52) (end 214.620136 96.52) (width 1.27) (layer F.Cu) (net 13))
 (segment (start 214.620136 96.52) (end 211.445136 99.695) (width 1.27) (layer F.Cu) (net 13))
 (segment (start 211.445136 99.695) (end 163.656262 99.695) (width 1.27) (layer F.Cu) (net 13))
 (segment (start 123.19 110.49) (end 123.19 111.603551) (width 1.27) (layer F.Cu) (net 13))
 (segment (start 123.19 111.603551) (end 124.010912 112.424463) (width 1.27) (layer F.Cu) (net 13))
 (segment (start 124.010912 112.424463) (end 150.926799 112.424463) (width 1.27) (layer F.Cu) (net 13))
 (segment (start 150.926799 112.424463) (end 163.656262 99.695) (width 1.27) (layer F.Cu) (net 13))
 (segment (start 144.78 96.52) (end 142.24 93.98) (width 1.27) (layer B.Cu) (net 13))
 (segment (start 118.11 110.49) (end 118.11 111.603551) (width 1.27) (layer F.Cu) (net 13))
 (segment (start 118.11 111.603551) (end 118.62205 112.115601) (width 1.27) (layer F.Cu) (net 13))
 (segment (start 118.62205 112.115601) (end 121.564399 112.115601) (width 1.27) (layer F.Cu) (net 13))
 (segment (start 121.564399 112.115601) (end 122.402601 111.277399) (width 1.27) (layer F.Cu) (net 13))
 (segment (start 122.402601 111.277399) (end 123.19 110.49) (width 1.27) (layer F.Cu) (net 13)))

